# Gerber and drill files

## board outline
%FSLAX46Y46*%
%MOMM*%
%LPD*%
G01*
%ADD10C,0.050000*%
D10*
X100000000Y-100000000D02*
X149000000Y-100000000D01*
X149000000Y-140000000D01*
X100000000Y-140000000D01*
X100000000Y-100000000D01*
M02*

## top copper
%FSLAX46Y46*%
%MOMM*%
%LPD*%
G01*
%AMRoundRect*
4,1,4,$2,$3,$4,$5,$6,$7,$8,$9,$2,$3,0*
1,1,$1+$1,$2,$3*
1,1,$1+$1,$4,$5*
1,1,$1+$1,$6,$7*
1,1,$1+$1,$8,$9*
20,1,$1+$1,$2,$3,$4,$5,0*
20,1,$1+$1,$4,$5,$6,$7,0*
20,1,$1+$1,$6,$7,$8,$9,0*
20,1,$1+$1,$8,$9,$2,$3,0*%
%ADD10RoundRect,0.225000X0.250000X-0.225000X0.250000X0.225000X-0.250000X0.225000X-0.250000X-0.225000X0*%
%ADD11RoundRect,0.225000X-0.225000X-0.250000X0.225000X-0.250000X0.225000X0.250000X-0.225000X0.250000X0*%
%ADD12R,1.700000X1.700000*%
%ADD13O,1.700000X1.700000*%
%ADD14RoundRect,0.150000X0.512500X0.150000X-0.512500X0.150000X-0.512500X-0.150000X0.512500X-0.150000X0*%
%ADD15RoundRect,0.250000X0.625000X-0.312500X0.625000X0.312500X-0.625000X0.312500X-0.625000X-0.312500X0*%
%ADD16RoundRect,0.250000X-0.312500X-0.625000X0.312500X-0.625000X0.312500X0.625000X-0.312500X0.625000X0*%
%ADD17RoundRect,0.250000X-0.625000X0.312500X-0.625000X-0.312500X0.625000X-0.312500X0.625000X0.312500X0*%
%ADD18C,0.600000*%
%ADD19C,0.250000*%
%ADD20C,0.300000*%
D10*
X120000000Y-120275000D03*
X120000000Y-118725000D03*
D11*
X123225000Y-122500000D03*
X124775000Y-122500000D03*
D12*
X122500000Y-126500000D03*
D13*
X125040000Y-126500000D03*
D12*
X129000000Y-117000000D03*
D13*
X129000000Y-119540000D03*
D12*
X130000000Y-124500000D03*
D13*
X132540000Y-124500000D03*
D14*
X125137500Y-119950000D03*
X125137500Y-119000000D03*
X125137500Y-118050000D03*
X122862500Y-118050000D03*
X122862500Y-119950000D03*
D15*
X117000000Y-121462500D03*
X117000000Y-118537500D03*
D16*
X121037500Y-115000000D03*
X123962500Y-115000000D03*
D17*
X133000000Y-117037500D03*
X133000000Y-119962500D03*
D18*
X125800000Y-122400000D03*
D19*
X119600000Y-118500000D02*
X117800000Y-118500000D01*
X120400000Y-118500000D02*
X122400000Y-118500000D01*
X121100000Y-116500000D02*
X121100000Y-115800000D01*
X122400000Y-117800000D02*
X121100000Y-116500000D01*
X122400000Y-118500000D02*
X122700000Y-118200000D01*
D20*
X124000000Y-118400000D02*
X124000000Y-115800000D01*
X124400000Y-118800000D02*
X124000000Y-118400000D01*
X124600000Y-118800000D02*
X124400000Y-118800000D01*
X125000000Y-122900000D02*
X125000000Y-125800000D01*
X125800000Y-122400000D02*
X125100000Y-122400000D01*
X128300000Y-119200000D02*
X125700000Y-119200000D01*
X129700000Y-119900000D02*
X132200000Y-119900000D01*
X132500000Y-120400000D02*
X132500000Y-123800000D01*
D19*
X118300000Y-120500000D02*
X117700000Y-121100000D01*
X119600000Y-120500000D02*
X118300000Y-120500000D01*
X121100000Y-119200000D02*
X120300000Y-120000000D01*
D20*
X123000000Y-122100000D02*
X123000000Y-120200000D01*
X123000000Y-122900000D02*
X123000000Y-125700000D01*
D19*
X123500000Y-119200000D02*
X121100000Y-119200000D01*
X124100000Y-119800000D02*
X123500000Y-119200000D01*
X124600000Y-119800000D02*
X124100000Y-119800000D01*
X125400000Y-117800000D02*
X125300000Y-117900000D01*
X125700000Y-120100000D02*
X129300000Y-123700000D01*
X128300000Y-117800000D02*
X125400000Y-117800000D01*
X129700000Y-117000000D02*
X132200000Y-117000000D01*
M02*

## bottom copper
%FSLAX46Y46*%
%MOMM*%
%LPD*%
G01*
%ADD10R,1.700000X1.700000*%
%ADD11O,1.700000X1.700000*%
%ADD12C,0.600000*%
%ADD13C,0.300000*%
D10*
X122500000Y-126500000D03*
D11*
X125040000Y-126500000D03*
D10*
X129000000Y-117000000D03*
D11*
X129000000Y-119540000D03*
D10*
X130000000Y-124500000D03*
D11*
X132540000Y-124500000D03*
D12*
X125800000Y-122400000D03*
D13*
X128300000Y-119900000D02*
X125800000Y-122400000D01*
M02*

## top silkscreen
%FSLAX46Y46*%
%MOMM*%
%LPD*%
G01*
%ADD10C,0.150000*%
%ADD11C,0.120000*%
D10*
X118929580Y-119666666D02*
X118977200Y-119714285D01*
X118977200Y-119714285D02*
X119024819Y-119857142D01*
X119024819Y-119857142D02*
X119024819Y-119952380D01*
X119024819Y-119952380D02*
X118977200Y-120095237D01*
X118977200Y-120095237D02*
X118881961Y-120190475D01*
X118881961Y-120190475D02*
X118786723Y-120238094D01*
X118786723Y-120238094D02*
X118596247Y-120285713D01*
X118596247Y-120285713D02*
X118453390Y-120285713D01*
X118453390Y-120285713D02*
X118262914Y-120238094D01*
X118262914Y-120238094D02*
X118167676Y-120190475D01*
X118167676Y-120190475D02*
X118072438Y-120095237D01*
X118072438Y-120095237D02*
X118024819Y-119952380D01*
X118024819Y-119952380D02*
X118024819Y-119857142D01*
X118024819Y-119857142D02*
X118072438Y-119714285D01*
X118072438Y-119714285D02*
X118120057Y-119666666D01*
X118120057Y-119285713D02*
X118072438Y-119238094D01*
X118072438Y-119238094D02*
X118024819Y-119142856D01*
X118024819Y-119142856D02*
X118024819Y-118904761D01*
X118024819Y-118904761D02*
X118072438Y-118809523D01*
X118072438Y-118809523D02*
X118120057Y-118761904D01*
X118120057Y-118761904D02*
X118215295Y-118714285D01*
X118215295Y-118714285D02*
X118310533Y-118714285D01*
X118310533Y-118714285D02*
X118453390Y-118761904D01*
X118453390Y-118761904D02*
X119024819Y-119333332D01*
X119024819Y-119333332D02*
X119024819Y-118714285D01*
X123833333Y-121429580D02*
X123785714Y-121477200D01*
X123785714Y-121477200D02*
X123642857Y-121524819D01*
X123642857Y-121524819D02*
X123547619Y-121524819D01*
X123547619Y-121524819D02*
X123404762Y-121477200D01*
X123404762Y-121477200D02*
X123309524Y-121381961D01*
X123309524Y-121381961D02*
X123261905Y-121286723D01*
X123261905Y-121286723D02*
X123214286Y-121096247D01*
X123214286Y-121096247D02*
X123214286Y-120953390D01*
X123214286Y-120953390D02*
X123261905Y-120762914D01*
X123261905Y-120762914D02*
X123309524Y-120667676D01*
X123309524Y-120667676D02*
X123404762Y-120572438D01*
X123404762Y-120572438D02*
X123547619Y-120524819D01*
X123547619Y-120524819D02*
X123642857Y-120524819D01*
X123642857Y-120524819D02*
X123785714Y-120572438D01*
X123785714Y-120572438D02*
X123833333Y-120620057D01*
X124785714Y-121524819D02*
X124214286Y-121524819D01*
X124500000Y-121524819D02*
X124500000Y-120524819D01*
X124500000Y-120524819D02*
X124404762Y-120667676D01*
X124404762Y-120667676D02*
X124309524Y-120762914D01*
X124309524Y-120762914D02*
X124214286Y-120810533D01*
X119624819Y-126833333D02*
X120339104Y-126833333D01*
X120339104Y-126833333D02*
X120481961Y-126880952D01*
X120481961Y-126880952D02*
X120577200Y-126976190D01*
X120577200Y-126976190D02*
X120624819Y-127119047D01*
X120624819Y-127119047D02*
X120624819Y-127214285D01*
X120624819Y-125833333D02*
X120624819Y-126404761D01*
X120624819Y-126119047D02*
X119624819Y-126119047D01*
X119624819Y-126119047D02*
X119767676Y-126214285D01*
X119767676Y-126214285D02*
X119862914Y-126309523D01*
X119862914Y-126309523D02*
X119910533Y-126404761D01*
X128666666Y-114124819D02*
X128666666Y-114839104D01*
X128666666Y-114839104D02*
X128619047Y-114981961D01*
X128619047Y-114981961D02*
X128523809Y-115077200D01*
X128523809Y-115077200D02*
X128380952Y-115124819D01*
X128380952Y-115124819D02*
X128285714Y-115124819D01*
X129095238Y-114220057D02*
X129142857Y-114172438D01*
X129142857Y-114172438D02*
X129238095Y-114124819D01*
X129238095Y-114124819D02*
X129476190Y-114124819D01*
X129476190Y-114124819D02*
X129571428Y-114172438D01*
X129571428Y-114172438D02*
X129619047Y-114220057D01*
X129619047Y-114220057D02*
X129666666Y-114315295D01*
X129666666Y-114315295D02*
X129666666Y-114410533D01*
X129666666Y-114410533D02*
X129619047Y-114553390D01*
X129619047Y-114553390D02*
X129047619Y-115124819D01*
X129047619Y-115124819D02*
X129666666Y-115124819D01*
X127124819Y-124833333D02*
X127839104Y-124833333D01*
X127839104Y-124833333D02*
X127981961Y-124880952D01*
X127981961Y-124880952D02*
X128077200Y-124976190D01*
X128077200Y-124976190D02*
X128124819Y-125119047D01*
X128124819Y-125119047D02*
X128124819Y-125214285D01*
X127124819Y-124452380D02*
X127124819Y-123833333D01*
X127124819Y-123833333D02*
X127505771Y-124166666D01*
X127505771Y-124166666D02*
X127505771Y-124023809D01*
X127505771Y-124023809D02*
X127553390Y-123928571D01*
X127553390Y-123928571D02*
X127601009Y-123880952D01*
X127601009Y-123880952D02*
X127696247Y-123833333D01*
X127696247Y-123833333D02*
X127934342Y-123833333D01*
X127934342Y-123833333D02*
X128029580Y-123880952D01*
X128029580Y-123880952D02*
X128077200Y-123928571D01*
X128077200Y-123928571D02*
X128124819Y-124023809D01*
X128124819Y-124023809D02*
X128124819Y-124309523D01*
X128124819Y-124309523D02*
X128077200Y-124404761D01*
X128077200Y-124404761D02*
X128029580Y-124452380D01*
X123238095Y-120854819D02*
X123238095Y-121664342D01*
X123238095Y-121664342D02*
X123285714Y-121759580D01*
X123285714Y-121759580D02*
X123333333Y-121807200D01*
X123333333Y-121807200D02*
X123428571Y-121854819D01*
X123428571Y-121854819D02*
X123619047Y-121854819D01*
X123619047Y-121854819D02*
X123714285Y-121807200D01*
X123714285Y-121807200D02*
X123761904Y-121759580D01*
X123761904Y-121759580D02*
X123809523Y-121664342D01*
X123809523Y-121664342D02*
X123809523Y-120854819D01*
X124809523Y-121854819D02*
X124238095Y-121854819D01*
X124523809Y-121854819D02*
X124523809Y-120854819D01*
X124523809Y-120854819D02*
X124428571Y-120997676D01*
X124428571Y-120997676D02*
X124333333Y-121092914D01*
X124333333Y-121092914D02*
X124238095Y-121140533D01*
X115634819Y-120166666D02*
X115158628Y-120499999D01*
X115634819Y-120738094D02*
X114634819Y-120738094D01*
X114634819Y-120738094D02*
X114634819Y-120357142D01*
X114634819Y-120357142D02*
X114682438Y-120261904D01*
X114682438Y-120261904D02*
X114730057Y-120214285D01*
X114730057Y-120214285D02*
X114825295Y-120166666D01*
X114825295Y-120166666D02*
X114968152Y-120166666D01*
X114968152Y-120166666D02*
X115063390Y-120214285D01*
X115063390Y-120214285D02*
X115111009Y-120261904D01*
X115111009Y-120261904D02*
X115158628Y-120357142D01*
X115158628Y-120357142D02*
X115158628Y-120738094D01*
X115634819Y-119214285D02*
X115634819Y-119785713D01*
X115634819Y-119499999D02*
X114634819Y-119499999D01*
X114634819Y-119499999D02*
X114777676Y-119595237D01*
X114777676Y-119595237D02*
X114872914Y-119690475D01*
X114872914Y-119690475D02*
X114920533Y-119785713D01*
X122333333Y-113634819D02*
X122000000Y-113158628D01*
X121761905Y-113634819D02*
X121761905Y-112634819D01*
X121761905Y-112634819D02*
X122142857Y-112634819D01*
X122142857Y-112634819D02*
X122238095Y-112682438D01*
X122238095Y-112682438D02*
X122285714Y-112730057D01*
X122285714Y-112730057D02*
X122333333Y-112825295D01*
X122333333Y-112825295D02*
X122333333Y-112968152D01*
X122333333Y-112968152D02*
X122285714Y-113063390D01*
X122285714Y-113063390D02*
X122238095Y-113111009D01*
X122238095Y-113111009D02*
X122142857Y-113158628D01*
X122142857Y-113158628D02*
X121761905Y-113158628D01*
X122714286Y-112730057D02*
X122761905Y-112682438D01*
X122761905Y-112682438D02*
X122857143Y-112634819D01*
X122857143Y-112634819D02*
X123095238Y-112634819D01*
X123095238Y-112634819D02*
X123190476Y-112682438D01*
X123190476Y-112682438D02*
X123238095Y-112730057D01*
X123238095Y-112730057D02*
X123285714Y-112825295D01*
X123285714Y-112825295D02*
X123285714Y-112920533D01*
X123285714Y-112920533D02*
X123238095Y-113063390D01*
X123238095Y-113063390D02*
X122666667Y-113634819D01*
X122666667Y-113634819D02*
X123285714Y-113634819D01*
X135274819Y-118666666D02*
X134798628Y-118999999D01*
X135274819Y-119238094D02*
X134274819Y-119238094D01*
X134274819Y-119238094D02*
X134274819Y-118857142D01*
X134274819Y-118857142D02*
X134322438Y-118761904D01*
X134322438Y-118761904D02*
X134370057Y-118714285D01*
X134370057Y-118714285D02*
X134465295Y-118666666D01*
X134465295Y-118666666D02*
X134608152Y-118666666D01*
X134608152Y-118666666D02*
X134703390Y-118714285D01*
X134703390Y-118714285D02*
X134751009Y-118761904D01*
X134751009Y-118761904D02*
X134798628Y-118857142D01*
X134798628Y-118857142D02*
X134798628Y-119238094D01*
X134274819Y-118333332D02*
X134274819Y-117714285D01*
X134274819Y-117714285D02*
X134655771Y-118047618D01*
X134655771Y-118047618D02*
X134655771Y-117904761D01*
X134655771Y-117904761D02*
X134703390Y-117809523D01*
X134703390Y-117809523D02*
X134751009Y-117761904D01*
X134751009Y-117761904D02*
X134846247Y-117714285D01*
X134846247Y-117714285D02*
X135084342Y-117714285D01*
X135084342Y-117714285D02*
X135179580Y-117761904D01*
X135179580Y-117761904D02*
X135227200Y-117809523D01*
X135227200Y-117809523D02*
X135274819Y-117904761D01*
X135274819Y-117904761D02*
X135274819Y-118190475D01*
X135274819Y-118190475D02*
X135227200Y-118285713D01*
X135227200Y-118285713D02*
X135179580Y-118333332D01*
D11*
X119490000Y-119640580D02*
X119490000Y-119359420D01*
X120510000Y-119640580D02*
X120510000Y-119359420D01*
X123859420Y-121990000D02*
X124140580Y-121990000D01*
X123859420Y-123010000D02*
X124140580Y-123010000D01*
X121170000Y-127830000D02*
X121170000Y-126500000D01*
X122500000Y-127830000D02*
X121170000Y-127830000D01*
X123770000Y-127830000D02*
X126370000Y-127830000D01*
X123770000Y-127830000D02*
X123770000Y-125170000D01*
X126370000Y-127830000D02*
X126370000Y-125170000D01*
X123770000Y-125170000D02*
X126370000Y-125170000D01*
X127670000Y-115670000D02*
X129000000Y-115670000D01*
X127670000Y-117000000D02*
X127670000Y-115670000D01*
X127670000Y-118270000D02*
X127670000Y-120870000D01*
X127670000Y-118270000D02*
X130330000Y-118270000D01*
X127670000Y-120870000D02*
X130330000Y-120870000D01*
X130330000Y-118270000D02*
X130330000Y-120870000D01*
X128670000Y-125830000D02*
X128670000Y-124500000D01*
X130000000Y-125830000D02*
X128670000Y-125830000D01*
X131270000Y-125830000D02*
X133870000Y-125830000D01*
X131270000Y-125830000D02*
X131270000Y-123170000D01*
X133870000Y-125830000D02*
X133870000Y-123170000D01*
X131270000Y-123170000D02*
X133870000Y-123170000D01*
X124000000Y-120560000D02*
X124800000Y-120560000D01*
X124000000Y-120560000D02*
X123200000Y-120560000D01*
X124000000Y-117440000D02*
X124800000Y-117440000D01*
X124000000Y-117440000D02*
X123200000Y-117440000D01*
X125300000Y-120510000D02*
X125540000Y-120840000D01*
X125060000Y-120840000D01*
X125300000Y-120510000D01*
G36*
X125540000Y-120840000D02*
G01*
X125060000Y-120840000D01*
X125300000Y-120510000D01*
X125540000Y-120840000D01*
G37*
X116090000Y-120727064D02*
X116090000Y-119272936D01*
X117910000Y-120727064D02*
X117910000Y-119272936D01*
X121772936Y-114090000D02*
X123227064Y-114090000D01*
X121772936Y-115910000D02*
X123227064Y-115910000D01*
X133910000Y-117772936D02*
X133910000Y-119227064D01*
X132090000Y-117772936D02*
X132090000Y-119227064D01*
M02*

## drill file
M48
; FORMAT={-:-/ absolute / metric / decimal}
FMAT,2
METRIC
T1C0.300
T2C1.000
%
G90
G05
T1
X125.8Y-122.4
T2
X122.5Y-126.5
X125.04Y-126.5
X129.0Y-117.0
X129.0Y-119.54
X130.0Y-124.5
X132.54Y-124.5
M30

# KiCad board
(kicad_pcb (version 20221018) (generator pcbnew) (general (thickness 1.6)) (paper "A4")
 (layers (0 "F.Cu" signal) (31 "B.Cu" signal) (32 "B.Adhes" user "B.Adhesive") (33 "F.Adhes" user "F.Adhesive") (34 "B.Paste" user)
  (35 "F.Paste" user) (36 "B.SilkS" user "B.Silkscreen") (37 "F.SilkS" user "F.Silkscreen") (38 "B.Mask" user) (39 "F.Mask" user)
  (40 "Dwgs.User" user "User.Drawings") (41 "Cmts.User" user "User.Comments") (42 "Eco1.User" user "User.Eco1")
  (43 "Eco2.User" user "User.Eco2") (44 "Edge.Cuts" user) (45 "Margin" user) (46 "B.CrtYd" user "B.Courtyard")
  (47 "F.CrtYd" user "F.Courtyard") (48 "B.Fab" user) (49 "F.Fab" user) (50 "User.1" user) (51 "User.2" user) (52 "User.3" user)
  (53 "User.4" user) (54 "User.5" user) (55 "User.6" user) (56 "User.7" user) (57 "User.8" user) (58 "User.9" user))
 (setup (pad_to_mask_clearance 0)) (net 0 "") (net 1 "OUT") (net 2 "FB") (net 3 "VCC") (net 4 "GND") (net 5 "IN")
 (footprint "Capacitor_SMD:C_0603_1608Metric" (layer "F.Cu") (at 120 119.5 90)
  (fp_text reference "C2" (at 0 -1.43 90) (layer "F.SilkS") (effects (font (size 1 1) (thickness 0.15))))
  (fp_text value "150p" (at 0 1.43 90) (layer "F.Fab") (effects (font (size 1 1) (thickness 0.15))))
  (fp_line (start -0.14058 -0.51) (end 0.14058 -0.51) (stroke (width 0.12) (type solid)) (layer "F.SilkS"))
  (fp_line (start -0.14058 0.51) (end 0.14058 0.51) (stroke (width 0.12) (type solid)) (layer "F.SilkS"))
  (pad "1" smd roundrect (at -0.775 0 90) (size 0.9 0.95) (layers "F.Cu" "F.Paste" "F.Mask") (roundrect_rratio 0.25) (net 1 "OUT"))
  (pad "2" smd roundrect (at 0.775 0 90) (size 0.9 0.95) (layers "F.Cu" "F.Paste" "F.Mask") (roundrect_rratio 0.25) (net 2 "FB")))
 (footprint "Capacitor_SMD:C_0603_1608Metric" (layer "F.Cu") (at 124 122.5)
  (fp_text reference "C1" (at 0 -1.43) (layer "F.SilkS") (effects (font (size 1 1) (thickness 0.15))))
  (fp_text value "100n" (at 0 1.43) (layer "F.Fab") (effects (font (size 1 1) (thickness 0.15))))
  (fp_line (start -0.14058 -0.51) (end 0.14058 -0.51) (stroke (width 0.12) (type solid)) (layer "F.SilkS"))
  (fp_line (start -0.14058 0.51) (end 0.14058 0.51) (stroke (width 0.12) (type solid)) (layer "F.SilkS"))
  (pad "1" smd roundrect (at -0.775 0) (size 0.9 0.95) (layers "F.Cu" "F.Paste" "F.Mask") (roundrect_rratio 0.25) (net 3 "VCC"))
  (pad "2" smd roundrect (at 0.775 0) (size 0.9 0.95) (layers "F.Cu" "F.Paste" "F.Mask") (roundrect_rratio 0.25) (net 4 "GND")))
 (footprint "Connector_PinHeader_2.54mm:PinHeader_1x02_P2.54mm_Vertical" (layer "F.Cu") (at 122.5 126.5 90)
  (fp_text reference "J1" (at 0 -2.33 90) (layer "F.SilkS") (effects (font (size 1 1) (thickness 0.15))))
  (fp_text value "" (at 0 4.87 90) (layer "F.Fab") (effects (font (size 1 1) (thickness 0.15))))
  (fp_line (start -1.33 -1.33) (end 0 -1.33) (stroke (width 0.12) (type solid)) (layer "F.SilkS"))
  (fp_line (start -1.33 0) (end -1.33 -1.33) (stroke (width 0.12) (type solid)) (layer "F.SilkS"))
  (fp_line (start -1.33 1.27) (end -1.33 3.87) (stroke (width 0.12) (type solid)) (layer "F.SilkS"))
  (fp_line (start -1.33 1.27) (end 1.33 1.27) (stroke (width 0.12) (type solid)) (layer "F.SilkS"))
  (fp_line (start -1.33 3.87) (end 1.33 3.87) (stroke (width 0.12) (type solid)) (layer "F.SilkS"))
  (fp_line (start 1.33 1.27) (end 1.33 3.87) (stroke (width 0.12) (type solid)) (layer "F.SilkS"))
  (pad "1" thru_hole rect (at 0 0 90) (size 1.7 1.7) (drill 1) (layers "*.Cu" "*.Mask") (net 3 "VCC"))
  (pad "2" thru_hole oval (at 0 2.54 90) (size 1.7 1.7) (drill 1) (layers "*.Cu" "*.Mask") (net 4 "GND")))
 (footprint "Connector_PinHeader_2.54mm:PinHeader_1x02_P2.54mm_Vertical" (layer "F.Cu") (at 129 117)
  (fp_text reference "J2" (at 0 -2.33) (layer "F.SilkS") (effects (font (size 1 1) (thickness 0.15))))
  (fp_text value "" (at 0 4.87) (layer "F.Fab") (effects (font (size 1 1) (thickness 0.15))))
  (fp_line (start -1.33 -1.33) (end 0 -1.33) (stroke (width 0.12) (type solid)) (layer "F.SilkS"))
  (fp_line (start -1.33 0) (end -1.33 -1.33) (stroke (width 0.12) (type solid)) (layer "F.SilkS"))
  (fp_line (start -1.33 1.27) (end -1.33 3.87) (stroke (width 0.12) (type solid)) (layer "F.SilkS"))
  (fp_line (start -1.33 1.27) (end 1.33 1.27) (stroke (width 0.12) (type solid)) (layer "F.SilkS"))
  (fp_line (start -1.33 3.87) (end 1.33 3.87) (stroke (width 0.12) (type solid)) (layer "F.SilkS"))
  (fp_line (start 1.33 1.27) (end 1.33 3.87) (stroke (width 0.12) (type solid)) (layer "F.SilkS"))
  (pad "1" thru_hole rect (at 0 0) (size 1.7 1.7) (drill 1) (layers "*.Cu" "*.Mask") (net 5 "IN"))
  (pad "2" thru_hole oval (at 0 2.54) (size 1.7 1.7) (drill 1) (layers "*.Cu" "*.Mask") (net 4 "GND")))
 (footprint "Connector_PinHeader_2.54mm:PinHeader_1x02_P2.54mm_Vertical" (layer "F.Cu") (at 130 124.5 90)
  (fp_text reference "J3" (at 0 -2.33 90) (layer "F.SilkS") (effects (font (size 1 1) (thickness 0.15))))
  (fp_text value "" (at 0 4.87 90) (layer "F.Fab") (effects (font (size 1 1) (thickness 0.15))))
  (fp_line (start -1.33 -1.33) (end 0 -1.33) (stroke (width 0.12) (type solid)) (layer "F.SilkS"))
  (fp_line (start -1.33 0) (end -1.33 -1.33) (stroke (width 0.12) (type solid)) (layer "F.SilkS"))
  (fp_line (start -1.33 1.27) (end -1.33 3.87) (stroke (width 0.12) (type solid)) (layer "F.SilkS"))
  (fp_line (start -1.33 1.27) (end 1.33 1.27) (stroke (width 0.12) (type solid)) (layer "F.SilkS"))
  (fp_line (start -1.33 3.87) (end 1.33 3.87) (stroke (width 0.12) (type solid)) (layer "F.SilkS"))
  (fp_line (start 1.33 1.27) (end 1.33 3.87) (stroke (width 0.12) (type solid)) (layer "F.SilkS"))
  (pad "1" thru_hole rect (at 0 0 90) (size 1.7 1.7) (drill 1) (layers "*.Cu" "*.Mask") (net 1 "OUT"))
  (pad "2" thru_hole oval (at 0 2.54 90) (size 1.7 1.7) (drill 1) (layers "*.Cu" "*.Mask") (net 4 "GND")))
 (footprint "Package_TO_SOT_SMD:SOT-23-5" (layer "F.Cu") (at 124 119 180)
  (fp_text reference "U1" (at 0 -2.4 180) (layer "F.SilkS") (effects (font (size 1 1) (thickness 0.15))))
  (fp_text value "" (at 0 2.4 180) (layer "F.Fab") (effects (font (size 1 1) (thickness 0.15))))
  (fp_line (start 0 -1.56) (end -0.8 -1.56) (stroke (width 0.12) (type solid)) (layer "F.SilkS"))
  (fp_line (start 0 -1.56) (end 0.8 -1.56) (stroke (width 0.12) (type solid)) (layer "F.SilkS"))
  (fp_line (start 0 1.56) (end -0.8 1.56) (stroke (width 0.12) (type solid)) (layer "F.SilkS"))
  (fp_line (start 0 1.56) (end 0.8 1.56) (stroke (width 0.12) (type solid)) (layer "F.SilkS"))
  (fp_poly
   (pts (xy -1.3 -1.51) (xy -1.54 -1.84) (xy -1.06 -1.84) (xy -1.3 -1.51)) (stroke (width 0.12) (type solid)) (fill solid) (layer "F.SilkS"))
  (pad "1" smd roundrect (at -1.1375 -0.95 180) (size 1.325 0.6) (layers "F.Cu" "F.Paste" "F.Mask") (roundrect_rratio 0.25) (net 1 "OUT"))
  (pad "2" smd roundrect (at -1.1375 0 180) (size 1.325 0.6) (layers "F.Cu" "F.Paste" "F.Mask") (roundrect_rratio 0.25) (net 4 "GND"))
  (pad "3" smd roundrect (at -1.1375 0.95 180) (size 1.325 0.6) (layers "F.Cu" "F.Paste" "F.Mask") (roundrect_rratio 0.25) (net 5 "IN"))
  (pad "4" smd roundrect (at 1.1375 0.95 180) (size 1.325 0.6) (layers "F.Cu" "F.Paste" "F.Mask") (roundrect_rratio 0.25) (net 2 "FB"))
  (pad "5" smd roundrect (at 1.1375 -0.95 180) (size 1.325 0.6) (layers "F.Cu" "F.Paste" "F.Mask") (roundrect_rratio 0.25) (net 3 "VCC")))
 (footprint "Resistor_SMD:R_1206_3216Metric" (layer "F.Cu") (at 117 120 90)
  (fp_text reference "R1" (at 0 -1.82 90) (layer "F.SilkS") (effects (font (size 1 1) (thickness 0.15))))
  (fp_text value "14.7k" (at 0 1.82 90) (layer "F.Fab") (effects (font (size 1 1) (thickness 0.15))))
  (fp_line (start -0.727064 -0.91) (end 0.727064 -0.91) (stroke (width 0.12) (type solid)) (layer "F.SilkS"))
  (fp_line (start -0.727064 0.91) (end 0.727064 0.91) (stroke (width 0.12) (type solid)) (layer "F.SilkS"))
  (pad "1" smd roundrect (at -1.4625 0 90) (size 1.125 1.75) (layers "F.Cu" "F.Paste" "F.Mask") (roundrect_rratio 0.222222) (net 1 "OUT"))
  (pad "2" smd roundrect (at 1.4625 0 90) (size 1.125 1.75) (layers "F.Cu" "F.Paste" "F.Mask") (roundrect_rratio 0.222222) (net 2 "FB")))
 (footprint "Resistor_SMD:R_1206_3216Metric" (layer "F.Cu") (at 122.5 115)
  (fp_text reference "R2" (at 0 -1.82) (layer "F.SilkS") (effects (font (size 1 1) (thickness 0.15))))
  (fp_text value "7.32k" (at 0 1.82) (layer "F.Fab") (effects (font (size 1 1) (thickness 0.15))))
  (fp_line (start -0.727064 -0.91) (end 0.727064 -0.91) (stroke (width 0.12) (type solid)) (layer "F.SilkS"))
  (fp_line (start -0.727064 0.91) (end 0.727064 0.91) (stroke (width 0.12) (type solid)) (layer "F.SilkS"))
  (pad "1" smd roundrect (at -1.4625 0) (size 1.125 1.75) (layers "F.Cu" "F.Paste" "F.Mask") (roundrect_rratio 0.222222) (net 2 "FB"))
  (pad "2" smd roundrect (at 1.4625 0) (size 1.125 1.75) (layers "F.Cu" "F.Paste" "F.Mask") (roundrect_rratio 0.222222) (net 4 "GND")))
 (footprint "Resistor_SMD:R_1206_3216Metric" (layer "F.Cu") (at 133 118.5 -90)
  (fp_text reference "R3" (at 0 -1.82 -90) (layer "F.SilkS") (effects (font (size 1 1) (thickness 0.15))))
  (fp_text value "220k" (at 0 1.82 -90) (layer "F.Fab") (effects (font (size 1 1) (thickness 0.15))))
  (fp_line (start -0.727064 -0.91) (end 0.727064 -0.91) (stroke (width 0.12) (type solid)) (layer "F.SilkS"))
  (fp_line (start -0.727064 0.91) (end 0.727064 0.91) (stroke (width 0.12) (type solid)) (layer "F.SilkS"))
  (pad "1" smd roundrect (at -1.4625 0 270) (size 1.125 1.75) (layers "F.Cu" "F.Paste" "F.Mask") (roundrect_rratio 0.222222) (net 5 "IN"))
  (pad "2" smd roundrect (at 1.4625 0 270) (size 1.125 1.75) (layers "F.Cu" "F.Paste" "F.Mask") (roundrect_rratio 0.222222) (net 4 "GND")))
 (gr_rect (start 100 100) (end 149 140) (stroke (width 0.05) (type default)) (fill none) (layer "Edge.Cuts"))
 (segment (start 119.6 118.5) (end 117.8 118.5) (width 0.25) (layer "F.Cu") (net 2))
 (segment (start 120.4 118.5) (end 122.4 118.5) (width 0.25) (layer "F.Cu") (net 2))
 (segment (start 121.1 116.5) (end 121.1 115.8) (width 0.25) (layer "F.Cu") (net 2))
 (segment (start 122.4 117.8) (end 121.1 116.5) (width 0.25) (layer "F.Cu") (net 2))
 (segment (start 122.4 118.5) (end 122.7 118.2) (width 0.25) (layer "F.Cu") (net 2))
 (segment (start 124 118.4) (end 124 115.8) (width 0.3) (layer "F.Cu") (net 4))
 (segment (start 124.4 118.8) (end 124 118.4) (width 0.3) (layer "F.Cu") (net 4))
 (segment (start 124.6 118.8) (end 124.4 118.8) (width 0.3) (layer "F.Cu") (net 4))
 (segment (start 125 122.9) (end 125 125.8) (width 0.3) (layer "F.Cu") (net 4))
 (segment (start 125.8 122.4) (end 125.1 122.4) (width 0.3) (layer "F.Cu") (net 4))
 (segment (start 128.3 119.2) (end 125.7 119.2) (width 0.3) (layer "F.Cu") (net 4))
 (segment (start 129.7 119.9) (end 132.2 119.9) (width 0.3) (layer "F.Cu") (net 4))
 (segment (start 132.5 120.4) (end 132.5 123.8) (width 0.3) (layer "F.Cu") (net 4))
 (via (at 125.8 122.4) (size 0.6) (drill 0.3) (layers "F.Cu" "B.Cu") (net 4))
 (segment (start 118.3 120.5) (end 117.7 121.1) (width 0.25) (layer "F.Cu") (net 1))
 (segment (start 119.6 120.5) (end 118.3 120.5) (width 0.25) (layer "F.Cu") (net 1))
 (segment (start 121.1 119.2) (end 120.3 120) (width 0.25) (layer "F.Cu") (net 1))
 (segment (start 123 122.1) (end 123 120.2) (width 0.3) (layer "F.Cu") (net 3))
 (segment (start 123 122.9) (end 123 125.7) (width 0.3) (layer "F.Cu") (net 3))
 (segment (start 123.5 119.2) (end 121.1 119.2) (width 0.25) (layer "F.Cu") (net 1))
 (segment (start 124.1 119.8) (end 123.5 119.2) (width 0.25) (layer "F.Cu") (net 1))
 (segment (start 124.6 119.8) (end 124.1 119.8) (width 0.25) (layer "F.Cu") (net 1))
 (segment (start 125.4 117.8) (end 125.3 117.9) (width 0.25) (layer "F.Cu") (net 5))
 (segment (start 125.7 120.1) (end 129.3 123.7) (width 0.25) (layer "F.Cu") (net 1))
 (segment (start 128.3 117.8) (end 125.4 117.8) (width 0.25) (layer "F.Cu") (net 5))
 (segment (start 128.3 119.9) (end 125.8 122.4) (width 0.3) (layer "B.Cu") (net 4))
 (segment (start 129.7 117) (end 132.2 117) (width 0.25) (layer "F.Cu") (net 5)))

